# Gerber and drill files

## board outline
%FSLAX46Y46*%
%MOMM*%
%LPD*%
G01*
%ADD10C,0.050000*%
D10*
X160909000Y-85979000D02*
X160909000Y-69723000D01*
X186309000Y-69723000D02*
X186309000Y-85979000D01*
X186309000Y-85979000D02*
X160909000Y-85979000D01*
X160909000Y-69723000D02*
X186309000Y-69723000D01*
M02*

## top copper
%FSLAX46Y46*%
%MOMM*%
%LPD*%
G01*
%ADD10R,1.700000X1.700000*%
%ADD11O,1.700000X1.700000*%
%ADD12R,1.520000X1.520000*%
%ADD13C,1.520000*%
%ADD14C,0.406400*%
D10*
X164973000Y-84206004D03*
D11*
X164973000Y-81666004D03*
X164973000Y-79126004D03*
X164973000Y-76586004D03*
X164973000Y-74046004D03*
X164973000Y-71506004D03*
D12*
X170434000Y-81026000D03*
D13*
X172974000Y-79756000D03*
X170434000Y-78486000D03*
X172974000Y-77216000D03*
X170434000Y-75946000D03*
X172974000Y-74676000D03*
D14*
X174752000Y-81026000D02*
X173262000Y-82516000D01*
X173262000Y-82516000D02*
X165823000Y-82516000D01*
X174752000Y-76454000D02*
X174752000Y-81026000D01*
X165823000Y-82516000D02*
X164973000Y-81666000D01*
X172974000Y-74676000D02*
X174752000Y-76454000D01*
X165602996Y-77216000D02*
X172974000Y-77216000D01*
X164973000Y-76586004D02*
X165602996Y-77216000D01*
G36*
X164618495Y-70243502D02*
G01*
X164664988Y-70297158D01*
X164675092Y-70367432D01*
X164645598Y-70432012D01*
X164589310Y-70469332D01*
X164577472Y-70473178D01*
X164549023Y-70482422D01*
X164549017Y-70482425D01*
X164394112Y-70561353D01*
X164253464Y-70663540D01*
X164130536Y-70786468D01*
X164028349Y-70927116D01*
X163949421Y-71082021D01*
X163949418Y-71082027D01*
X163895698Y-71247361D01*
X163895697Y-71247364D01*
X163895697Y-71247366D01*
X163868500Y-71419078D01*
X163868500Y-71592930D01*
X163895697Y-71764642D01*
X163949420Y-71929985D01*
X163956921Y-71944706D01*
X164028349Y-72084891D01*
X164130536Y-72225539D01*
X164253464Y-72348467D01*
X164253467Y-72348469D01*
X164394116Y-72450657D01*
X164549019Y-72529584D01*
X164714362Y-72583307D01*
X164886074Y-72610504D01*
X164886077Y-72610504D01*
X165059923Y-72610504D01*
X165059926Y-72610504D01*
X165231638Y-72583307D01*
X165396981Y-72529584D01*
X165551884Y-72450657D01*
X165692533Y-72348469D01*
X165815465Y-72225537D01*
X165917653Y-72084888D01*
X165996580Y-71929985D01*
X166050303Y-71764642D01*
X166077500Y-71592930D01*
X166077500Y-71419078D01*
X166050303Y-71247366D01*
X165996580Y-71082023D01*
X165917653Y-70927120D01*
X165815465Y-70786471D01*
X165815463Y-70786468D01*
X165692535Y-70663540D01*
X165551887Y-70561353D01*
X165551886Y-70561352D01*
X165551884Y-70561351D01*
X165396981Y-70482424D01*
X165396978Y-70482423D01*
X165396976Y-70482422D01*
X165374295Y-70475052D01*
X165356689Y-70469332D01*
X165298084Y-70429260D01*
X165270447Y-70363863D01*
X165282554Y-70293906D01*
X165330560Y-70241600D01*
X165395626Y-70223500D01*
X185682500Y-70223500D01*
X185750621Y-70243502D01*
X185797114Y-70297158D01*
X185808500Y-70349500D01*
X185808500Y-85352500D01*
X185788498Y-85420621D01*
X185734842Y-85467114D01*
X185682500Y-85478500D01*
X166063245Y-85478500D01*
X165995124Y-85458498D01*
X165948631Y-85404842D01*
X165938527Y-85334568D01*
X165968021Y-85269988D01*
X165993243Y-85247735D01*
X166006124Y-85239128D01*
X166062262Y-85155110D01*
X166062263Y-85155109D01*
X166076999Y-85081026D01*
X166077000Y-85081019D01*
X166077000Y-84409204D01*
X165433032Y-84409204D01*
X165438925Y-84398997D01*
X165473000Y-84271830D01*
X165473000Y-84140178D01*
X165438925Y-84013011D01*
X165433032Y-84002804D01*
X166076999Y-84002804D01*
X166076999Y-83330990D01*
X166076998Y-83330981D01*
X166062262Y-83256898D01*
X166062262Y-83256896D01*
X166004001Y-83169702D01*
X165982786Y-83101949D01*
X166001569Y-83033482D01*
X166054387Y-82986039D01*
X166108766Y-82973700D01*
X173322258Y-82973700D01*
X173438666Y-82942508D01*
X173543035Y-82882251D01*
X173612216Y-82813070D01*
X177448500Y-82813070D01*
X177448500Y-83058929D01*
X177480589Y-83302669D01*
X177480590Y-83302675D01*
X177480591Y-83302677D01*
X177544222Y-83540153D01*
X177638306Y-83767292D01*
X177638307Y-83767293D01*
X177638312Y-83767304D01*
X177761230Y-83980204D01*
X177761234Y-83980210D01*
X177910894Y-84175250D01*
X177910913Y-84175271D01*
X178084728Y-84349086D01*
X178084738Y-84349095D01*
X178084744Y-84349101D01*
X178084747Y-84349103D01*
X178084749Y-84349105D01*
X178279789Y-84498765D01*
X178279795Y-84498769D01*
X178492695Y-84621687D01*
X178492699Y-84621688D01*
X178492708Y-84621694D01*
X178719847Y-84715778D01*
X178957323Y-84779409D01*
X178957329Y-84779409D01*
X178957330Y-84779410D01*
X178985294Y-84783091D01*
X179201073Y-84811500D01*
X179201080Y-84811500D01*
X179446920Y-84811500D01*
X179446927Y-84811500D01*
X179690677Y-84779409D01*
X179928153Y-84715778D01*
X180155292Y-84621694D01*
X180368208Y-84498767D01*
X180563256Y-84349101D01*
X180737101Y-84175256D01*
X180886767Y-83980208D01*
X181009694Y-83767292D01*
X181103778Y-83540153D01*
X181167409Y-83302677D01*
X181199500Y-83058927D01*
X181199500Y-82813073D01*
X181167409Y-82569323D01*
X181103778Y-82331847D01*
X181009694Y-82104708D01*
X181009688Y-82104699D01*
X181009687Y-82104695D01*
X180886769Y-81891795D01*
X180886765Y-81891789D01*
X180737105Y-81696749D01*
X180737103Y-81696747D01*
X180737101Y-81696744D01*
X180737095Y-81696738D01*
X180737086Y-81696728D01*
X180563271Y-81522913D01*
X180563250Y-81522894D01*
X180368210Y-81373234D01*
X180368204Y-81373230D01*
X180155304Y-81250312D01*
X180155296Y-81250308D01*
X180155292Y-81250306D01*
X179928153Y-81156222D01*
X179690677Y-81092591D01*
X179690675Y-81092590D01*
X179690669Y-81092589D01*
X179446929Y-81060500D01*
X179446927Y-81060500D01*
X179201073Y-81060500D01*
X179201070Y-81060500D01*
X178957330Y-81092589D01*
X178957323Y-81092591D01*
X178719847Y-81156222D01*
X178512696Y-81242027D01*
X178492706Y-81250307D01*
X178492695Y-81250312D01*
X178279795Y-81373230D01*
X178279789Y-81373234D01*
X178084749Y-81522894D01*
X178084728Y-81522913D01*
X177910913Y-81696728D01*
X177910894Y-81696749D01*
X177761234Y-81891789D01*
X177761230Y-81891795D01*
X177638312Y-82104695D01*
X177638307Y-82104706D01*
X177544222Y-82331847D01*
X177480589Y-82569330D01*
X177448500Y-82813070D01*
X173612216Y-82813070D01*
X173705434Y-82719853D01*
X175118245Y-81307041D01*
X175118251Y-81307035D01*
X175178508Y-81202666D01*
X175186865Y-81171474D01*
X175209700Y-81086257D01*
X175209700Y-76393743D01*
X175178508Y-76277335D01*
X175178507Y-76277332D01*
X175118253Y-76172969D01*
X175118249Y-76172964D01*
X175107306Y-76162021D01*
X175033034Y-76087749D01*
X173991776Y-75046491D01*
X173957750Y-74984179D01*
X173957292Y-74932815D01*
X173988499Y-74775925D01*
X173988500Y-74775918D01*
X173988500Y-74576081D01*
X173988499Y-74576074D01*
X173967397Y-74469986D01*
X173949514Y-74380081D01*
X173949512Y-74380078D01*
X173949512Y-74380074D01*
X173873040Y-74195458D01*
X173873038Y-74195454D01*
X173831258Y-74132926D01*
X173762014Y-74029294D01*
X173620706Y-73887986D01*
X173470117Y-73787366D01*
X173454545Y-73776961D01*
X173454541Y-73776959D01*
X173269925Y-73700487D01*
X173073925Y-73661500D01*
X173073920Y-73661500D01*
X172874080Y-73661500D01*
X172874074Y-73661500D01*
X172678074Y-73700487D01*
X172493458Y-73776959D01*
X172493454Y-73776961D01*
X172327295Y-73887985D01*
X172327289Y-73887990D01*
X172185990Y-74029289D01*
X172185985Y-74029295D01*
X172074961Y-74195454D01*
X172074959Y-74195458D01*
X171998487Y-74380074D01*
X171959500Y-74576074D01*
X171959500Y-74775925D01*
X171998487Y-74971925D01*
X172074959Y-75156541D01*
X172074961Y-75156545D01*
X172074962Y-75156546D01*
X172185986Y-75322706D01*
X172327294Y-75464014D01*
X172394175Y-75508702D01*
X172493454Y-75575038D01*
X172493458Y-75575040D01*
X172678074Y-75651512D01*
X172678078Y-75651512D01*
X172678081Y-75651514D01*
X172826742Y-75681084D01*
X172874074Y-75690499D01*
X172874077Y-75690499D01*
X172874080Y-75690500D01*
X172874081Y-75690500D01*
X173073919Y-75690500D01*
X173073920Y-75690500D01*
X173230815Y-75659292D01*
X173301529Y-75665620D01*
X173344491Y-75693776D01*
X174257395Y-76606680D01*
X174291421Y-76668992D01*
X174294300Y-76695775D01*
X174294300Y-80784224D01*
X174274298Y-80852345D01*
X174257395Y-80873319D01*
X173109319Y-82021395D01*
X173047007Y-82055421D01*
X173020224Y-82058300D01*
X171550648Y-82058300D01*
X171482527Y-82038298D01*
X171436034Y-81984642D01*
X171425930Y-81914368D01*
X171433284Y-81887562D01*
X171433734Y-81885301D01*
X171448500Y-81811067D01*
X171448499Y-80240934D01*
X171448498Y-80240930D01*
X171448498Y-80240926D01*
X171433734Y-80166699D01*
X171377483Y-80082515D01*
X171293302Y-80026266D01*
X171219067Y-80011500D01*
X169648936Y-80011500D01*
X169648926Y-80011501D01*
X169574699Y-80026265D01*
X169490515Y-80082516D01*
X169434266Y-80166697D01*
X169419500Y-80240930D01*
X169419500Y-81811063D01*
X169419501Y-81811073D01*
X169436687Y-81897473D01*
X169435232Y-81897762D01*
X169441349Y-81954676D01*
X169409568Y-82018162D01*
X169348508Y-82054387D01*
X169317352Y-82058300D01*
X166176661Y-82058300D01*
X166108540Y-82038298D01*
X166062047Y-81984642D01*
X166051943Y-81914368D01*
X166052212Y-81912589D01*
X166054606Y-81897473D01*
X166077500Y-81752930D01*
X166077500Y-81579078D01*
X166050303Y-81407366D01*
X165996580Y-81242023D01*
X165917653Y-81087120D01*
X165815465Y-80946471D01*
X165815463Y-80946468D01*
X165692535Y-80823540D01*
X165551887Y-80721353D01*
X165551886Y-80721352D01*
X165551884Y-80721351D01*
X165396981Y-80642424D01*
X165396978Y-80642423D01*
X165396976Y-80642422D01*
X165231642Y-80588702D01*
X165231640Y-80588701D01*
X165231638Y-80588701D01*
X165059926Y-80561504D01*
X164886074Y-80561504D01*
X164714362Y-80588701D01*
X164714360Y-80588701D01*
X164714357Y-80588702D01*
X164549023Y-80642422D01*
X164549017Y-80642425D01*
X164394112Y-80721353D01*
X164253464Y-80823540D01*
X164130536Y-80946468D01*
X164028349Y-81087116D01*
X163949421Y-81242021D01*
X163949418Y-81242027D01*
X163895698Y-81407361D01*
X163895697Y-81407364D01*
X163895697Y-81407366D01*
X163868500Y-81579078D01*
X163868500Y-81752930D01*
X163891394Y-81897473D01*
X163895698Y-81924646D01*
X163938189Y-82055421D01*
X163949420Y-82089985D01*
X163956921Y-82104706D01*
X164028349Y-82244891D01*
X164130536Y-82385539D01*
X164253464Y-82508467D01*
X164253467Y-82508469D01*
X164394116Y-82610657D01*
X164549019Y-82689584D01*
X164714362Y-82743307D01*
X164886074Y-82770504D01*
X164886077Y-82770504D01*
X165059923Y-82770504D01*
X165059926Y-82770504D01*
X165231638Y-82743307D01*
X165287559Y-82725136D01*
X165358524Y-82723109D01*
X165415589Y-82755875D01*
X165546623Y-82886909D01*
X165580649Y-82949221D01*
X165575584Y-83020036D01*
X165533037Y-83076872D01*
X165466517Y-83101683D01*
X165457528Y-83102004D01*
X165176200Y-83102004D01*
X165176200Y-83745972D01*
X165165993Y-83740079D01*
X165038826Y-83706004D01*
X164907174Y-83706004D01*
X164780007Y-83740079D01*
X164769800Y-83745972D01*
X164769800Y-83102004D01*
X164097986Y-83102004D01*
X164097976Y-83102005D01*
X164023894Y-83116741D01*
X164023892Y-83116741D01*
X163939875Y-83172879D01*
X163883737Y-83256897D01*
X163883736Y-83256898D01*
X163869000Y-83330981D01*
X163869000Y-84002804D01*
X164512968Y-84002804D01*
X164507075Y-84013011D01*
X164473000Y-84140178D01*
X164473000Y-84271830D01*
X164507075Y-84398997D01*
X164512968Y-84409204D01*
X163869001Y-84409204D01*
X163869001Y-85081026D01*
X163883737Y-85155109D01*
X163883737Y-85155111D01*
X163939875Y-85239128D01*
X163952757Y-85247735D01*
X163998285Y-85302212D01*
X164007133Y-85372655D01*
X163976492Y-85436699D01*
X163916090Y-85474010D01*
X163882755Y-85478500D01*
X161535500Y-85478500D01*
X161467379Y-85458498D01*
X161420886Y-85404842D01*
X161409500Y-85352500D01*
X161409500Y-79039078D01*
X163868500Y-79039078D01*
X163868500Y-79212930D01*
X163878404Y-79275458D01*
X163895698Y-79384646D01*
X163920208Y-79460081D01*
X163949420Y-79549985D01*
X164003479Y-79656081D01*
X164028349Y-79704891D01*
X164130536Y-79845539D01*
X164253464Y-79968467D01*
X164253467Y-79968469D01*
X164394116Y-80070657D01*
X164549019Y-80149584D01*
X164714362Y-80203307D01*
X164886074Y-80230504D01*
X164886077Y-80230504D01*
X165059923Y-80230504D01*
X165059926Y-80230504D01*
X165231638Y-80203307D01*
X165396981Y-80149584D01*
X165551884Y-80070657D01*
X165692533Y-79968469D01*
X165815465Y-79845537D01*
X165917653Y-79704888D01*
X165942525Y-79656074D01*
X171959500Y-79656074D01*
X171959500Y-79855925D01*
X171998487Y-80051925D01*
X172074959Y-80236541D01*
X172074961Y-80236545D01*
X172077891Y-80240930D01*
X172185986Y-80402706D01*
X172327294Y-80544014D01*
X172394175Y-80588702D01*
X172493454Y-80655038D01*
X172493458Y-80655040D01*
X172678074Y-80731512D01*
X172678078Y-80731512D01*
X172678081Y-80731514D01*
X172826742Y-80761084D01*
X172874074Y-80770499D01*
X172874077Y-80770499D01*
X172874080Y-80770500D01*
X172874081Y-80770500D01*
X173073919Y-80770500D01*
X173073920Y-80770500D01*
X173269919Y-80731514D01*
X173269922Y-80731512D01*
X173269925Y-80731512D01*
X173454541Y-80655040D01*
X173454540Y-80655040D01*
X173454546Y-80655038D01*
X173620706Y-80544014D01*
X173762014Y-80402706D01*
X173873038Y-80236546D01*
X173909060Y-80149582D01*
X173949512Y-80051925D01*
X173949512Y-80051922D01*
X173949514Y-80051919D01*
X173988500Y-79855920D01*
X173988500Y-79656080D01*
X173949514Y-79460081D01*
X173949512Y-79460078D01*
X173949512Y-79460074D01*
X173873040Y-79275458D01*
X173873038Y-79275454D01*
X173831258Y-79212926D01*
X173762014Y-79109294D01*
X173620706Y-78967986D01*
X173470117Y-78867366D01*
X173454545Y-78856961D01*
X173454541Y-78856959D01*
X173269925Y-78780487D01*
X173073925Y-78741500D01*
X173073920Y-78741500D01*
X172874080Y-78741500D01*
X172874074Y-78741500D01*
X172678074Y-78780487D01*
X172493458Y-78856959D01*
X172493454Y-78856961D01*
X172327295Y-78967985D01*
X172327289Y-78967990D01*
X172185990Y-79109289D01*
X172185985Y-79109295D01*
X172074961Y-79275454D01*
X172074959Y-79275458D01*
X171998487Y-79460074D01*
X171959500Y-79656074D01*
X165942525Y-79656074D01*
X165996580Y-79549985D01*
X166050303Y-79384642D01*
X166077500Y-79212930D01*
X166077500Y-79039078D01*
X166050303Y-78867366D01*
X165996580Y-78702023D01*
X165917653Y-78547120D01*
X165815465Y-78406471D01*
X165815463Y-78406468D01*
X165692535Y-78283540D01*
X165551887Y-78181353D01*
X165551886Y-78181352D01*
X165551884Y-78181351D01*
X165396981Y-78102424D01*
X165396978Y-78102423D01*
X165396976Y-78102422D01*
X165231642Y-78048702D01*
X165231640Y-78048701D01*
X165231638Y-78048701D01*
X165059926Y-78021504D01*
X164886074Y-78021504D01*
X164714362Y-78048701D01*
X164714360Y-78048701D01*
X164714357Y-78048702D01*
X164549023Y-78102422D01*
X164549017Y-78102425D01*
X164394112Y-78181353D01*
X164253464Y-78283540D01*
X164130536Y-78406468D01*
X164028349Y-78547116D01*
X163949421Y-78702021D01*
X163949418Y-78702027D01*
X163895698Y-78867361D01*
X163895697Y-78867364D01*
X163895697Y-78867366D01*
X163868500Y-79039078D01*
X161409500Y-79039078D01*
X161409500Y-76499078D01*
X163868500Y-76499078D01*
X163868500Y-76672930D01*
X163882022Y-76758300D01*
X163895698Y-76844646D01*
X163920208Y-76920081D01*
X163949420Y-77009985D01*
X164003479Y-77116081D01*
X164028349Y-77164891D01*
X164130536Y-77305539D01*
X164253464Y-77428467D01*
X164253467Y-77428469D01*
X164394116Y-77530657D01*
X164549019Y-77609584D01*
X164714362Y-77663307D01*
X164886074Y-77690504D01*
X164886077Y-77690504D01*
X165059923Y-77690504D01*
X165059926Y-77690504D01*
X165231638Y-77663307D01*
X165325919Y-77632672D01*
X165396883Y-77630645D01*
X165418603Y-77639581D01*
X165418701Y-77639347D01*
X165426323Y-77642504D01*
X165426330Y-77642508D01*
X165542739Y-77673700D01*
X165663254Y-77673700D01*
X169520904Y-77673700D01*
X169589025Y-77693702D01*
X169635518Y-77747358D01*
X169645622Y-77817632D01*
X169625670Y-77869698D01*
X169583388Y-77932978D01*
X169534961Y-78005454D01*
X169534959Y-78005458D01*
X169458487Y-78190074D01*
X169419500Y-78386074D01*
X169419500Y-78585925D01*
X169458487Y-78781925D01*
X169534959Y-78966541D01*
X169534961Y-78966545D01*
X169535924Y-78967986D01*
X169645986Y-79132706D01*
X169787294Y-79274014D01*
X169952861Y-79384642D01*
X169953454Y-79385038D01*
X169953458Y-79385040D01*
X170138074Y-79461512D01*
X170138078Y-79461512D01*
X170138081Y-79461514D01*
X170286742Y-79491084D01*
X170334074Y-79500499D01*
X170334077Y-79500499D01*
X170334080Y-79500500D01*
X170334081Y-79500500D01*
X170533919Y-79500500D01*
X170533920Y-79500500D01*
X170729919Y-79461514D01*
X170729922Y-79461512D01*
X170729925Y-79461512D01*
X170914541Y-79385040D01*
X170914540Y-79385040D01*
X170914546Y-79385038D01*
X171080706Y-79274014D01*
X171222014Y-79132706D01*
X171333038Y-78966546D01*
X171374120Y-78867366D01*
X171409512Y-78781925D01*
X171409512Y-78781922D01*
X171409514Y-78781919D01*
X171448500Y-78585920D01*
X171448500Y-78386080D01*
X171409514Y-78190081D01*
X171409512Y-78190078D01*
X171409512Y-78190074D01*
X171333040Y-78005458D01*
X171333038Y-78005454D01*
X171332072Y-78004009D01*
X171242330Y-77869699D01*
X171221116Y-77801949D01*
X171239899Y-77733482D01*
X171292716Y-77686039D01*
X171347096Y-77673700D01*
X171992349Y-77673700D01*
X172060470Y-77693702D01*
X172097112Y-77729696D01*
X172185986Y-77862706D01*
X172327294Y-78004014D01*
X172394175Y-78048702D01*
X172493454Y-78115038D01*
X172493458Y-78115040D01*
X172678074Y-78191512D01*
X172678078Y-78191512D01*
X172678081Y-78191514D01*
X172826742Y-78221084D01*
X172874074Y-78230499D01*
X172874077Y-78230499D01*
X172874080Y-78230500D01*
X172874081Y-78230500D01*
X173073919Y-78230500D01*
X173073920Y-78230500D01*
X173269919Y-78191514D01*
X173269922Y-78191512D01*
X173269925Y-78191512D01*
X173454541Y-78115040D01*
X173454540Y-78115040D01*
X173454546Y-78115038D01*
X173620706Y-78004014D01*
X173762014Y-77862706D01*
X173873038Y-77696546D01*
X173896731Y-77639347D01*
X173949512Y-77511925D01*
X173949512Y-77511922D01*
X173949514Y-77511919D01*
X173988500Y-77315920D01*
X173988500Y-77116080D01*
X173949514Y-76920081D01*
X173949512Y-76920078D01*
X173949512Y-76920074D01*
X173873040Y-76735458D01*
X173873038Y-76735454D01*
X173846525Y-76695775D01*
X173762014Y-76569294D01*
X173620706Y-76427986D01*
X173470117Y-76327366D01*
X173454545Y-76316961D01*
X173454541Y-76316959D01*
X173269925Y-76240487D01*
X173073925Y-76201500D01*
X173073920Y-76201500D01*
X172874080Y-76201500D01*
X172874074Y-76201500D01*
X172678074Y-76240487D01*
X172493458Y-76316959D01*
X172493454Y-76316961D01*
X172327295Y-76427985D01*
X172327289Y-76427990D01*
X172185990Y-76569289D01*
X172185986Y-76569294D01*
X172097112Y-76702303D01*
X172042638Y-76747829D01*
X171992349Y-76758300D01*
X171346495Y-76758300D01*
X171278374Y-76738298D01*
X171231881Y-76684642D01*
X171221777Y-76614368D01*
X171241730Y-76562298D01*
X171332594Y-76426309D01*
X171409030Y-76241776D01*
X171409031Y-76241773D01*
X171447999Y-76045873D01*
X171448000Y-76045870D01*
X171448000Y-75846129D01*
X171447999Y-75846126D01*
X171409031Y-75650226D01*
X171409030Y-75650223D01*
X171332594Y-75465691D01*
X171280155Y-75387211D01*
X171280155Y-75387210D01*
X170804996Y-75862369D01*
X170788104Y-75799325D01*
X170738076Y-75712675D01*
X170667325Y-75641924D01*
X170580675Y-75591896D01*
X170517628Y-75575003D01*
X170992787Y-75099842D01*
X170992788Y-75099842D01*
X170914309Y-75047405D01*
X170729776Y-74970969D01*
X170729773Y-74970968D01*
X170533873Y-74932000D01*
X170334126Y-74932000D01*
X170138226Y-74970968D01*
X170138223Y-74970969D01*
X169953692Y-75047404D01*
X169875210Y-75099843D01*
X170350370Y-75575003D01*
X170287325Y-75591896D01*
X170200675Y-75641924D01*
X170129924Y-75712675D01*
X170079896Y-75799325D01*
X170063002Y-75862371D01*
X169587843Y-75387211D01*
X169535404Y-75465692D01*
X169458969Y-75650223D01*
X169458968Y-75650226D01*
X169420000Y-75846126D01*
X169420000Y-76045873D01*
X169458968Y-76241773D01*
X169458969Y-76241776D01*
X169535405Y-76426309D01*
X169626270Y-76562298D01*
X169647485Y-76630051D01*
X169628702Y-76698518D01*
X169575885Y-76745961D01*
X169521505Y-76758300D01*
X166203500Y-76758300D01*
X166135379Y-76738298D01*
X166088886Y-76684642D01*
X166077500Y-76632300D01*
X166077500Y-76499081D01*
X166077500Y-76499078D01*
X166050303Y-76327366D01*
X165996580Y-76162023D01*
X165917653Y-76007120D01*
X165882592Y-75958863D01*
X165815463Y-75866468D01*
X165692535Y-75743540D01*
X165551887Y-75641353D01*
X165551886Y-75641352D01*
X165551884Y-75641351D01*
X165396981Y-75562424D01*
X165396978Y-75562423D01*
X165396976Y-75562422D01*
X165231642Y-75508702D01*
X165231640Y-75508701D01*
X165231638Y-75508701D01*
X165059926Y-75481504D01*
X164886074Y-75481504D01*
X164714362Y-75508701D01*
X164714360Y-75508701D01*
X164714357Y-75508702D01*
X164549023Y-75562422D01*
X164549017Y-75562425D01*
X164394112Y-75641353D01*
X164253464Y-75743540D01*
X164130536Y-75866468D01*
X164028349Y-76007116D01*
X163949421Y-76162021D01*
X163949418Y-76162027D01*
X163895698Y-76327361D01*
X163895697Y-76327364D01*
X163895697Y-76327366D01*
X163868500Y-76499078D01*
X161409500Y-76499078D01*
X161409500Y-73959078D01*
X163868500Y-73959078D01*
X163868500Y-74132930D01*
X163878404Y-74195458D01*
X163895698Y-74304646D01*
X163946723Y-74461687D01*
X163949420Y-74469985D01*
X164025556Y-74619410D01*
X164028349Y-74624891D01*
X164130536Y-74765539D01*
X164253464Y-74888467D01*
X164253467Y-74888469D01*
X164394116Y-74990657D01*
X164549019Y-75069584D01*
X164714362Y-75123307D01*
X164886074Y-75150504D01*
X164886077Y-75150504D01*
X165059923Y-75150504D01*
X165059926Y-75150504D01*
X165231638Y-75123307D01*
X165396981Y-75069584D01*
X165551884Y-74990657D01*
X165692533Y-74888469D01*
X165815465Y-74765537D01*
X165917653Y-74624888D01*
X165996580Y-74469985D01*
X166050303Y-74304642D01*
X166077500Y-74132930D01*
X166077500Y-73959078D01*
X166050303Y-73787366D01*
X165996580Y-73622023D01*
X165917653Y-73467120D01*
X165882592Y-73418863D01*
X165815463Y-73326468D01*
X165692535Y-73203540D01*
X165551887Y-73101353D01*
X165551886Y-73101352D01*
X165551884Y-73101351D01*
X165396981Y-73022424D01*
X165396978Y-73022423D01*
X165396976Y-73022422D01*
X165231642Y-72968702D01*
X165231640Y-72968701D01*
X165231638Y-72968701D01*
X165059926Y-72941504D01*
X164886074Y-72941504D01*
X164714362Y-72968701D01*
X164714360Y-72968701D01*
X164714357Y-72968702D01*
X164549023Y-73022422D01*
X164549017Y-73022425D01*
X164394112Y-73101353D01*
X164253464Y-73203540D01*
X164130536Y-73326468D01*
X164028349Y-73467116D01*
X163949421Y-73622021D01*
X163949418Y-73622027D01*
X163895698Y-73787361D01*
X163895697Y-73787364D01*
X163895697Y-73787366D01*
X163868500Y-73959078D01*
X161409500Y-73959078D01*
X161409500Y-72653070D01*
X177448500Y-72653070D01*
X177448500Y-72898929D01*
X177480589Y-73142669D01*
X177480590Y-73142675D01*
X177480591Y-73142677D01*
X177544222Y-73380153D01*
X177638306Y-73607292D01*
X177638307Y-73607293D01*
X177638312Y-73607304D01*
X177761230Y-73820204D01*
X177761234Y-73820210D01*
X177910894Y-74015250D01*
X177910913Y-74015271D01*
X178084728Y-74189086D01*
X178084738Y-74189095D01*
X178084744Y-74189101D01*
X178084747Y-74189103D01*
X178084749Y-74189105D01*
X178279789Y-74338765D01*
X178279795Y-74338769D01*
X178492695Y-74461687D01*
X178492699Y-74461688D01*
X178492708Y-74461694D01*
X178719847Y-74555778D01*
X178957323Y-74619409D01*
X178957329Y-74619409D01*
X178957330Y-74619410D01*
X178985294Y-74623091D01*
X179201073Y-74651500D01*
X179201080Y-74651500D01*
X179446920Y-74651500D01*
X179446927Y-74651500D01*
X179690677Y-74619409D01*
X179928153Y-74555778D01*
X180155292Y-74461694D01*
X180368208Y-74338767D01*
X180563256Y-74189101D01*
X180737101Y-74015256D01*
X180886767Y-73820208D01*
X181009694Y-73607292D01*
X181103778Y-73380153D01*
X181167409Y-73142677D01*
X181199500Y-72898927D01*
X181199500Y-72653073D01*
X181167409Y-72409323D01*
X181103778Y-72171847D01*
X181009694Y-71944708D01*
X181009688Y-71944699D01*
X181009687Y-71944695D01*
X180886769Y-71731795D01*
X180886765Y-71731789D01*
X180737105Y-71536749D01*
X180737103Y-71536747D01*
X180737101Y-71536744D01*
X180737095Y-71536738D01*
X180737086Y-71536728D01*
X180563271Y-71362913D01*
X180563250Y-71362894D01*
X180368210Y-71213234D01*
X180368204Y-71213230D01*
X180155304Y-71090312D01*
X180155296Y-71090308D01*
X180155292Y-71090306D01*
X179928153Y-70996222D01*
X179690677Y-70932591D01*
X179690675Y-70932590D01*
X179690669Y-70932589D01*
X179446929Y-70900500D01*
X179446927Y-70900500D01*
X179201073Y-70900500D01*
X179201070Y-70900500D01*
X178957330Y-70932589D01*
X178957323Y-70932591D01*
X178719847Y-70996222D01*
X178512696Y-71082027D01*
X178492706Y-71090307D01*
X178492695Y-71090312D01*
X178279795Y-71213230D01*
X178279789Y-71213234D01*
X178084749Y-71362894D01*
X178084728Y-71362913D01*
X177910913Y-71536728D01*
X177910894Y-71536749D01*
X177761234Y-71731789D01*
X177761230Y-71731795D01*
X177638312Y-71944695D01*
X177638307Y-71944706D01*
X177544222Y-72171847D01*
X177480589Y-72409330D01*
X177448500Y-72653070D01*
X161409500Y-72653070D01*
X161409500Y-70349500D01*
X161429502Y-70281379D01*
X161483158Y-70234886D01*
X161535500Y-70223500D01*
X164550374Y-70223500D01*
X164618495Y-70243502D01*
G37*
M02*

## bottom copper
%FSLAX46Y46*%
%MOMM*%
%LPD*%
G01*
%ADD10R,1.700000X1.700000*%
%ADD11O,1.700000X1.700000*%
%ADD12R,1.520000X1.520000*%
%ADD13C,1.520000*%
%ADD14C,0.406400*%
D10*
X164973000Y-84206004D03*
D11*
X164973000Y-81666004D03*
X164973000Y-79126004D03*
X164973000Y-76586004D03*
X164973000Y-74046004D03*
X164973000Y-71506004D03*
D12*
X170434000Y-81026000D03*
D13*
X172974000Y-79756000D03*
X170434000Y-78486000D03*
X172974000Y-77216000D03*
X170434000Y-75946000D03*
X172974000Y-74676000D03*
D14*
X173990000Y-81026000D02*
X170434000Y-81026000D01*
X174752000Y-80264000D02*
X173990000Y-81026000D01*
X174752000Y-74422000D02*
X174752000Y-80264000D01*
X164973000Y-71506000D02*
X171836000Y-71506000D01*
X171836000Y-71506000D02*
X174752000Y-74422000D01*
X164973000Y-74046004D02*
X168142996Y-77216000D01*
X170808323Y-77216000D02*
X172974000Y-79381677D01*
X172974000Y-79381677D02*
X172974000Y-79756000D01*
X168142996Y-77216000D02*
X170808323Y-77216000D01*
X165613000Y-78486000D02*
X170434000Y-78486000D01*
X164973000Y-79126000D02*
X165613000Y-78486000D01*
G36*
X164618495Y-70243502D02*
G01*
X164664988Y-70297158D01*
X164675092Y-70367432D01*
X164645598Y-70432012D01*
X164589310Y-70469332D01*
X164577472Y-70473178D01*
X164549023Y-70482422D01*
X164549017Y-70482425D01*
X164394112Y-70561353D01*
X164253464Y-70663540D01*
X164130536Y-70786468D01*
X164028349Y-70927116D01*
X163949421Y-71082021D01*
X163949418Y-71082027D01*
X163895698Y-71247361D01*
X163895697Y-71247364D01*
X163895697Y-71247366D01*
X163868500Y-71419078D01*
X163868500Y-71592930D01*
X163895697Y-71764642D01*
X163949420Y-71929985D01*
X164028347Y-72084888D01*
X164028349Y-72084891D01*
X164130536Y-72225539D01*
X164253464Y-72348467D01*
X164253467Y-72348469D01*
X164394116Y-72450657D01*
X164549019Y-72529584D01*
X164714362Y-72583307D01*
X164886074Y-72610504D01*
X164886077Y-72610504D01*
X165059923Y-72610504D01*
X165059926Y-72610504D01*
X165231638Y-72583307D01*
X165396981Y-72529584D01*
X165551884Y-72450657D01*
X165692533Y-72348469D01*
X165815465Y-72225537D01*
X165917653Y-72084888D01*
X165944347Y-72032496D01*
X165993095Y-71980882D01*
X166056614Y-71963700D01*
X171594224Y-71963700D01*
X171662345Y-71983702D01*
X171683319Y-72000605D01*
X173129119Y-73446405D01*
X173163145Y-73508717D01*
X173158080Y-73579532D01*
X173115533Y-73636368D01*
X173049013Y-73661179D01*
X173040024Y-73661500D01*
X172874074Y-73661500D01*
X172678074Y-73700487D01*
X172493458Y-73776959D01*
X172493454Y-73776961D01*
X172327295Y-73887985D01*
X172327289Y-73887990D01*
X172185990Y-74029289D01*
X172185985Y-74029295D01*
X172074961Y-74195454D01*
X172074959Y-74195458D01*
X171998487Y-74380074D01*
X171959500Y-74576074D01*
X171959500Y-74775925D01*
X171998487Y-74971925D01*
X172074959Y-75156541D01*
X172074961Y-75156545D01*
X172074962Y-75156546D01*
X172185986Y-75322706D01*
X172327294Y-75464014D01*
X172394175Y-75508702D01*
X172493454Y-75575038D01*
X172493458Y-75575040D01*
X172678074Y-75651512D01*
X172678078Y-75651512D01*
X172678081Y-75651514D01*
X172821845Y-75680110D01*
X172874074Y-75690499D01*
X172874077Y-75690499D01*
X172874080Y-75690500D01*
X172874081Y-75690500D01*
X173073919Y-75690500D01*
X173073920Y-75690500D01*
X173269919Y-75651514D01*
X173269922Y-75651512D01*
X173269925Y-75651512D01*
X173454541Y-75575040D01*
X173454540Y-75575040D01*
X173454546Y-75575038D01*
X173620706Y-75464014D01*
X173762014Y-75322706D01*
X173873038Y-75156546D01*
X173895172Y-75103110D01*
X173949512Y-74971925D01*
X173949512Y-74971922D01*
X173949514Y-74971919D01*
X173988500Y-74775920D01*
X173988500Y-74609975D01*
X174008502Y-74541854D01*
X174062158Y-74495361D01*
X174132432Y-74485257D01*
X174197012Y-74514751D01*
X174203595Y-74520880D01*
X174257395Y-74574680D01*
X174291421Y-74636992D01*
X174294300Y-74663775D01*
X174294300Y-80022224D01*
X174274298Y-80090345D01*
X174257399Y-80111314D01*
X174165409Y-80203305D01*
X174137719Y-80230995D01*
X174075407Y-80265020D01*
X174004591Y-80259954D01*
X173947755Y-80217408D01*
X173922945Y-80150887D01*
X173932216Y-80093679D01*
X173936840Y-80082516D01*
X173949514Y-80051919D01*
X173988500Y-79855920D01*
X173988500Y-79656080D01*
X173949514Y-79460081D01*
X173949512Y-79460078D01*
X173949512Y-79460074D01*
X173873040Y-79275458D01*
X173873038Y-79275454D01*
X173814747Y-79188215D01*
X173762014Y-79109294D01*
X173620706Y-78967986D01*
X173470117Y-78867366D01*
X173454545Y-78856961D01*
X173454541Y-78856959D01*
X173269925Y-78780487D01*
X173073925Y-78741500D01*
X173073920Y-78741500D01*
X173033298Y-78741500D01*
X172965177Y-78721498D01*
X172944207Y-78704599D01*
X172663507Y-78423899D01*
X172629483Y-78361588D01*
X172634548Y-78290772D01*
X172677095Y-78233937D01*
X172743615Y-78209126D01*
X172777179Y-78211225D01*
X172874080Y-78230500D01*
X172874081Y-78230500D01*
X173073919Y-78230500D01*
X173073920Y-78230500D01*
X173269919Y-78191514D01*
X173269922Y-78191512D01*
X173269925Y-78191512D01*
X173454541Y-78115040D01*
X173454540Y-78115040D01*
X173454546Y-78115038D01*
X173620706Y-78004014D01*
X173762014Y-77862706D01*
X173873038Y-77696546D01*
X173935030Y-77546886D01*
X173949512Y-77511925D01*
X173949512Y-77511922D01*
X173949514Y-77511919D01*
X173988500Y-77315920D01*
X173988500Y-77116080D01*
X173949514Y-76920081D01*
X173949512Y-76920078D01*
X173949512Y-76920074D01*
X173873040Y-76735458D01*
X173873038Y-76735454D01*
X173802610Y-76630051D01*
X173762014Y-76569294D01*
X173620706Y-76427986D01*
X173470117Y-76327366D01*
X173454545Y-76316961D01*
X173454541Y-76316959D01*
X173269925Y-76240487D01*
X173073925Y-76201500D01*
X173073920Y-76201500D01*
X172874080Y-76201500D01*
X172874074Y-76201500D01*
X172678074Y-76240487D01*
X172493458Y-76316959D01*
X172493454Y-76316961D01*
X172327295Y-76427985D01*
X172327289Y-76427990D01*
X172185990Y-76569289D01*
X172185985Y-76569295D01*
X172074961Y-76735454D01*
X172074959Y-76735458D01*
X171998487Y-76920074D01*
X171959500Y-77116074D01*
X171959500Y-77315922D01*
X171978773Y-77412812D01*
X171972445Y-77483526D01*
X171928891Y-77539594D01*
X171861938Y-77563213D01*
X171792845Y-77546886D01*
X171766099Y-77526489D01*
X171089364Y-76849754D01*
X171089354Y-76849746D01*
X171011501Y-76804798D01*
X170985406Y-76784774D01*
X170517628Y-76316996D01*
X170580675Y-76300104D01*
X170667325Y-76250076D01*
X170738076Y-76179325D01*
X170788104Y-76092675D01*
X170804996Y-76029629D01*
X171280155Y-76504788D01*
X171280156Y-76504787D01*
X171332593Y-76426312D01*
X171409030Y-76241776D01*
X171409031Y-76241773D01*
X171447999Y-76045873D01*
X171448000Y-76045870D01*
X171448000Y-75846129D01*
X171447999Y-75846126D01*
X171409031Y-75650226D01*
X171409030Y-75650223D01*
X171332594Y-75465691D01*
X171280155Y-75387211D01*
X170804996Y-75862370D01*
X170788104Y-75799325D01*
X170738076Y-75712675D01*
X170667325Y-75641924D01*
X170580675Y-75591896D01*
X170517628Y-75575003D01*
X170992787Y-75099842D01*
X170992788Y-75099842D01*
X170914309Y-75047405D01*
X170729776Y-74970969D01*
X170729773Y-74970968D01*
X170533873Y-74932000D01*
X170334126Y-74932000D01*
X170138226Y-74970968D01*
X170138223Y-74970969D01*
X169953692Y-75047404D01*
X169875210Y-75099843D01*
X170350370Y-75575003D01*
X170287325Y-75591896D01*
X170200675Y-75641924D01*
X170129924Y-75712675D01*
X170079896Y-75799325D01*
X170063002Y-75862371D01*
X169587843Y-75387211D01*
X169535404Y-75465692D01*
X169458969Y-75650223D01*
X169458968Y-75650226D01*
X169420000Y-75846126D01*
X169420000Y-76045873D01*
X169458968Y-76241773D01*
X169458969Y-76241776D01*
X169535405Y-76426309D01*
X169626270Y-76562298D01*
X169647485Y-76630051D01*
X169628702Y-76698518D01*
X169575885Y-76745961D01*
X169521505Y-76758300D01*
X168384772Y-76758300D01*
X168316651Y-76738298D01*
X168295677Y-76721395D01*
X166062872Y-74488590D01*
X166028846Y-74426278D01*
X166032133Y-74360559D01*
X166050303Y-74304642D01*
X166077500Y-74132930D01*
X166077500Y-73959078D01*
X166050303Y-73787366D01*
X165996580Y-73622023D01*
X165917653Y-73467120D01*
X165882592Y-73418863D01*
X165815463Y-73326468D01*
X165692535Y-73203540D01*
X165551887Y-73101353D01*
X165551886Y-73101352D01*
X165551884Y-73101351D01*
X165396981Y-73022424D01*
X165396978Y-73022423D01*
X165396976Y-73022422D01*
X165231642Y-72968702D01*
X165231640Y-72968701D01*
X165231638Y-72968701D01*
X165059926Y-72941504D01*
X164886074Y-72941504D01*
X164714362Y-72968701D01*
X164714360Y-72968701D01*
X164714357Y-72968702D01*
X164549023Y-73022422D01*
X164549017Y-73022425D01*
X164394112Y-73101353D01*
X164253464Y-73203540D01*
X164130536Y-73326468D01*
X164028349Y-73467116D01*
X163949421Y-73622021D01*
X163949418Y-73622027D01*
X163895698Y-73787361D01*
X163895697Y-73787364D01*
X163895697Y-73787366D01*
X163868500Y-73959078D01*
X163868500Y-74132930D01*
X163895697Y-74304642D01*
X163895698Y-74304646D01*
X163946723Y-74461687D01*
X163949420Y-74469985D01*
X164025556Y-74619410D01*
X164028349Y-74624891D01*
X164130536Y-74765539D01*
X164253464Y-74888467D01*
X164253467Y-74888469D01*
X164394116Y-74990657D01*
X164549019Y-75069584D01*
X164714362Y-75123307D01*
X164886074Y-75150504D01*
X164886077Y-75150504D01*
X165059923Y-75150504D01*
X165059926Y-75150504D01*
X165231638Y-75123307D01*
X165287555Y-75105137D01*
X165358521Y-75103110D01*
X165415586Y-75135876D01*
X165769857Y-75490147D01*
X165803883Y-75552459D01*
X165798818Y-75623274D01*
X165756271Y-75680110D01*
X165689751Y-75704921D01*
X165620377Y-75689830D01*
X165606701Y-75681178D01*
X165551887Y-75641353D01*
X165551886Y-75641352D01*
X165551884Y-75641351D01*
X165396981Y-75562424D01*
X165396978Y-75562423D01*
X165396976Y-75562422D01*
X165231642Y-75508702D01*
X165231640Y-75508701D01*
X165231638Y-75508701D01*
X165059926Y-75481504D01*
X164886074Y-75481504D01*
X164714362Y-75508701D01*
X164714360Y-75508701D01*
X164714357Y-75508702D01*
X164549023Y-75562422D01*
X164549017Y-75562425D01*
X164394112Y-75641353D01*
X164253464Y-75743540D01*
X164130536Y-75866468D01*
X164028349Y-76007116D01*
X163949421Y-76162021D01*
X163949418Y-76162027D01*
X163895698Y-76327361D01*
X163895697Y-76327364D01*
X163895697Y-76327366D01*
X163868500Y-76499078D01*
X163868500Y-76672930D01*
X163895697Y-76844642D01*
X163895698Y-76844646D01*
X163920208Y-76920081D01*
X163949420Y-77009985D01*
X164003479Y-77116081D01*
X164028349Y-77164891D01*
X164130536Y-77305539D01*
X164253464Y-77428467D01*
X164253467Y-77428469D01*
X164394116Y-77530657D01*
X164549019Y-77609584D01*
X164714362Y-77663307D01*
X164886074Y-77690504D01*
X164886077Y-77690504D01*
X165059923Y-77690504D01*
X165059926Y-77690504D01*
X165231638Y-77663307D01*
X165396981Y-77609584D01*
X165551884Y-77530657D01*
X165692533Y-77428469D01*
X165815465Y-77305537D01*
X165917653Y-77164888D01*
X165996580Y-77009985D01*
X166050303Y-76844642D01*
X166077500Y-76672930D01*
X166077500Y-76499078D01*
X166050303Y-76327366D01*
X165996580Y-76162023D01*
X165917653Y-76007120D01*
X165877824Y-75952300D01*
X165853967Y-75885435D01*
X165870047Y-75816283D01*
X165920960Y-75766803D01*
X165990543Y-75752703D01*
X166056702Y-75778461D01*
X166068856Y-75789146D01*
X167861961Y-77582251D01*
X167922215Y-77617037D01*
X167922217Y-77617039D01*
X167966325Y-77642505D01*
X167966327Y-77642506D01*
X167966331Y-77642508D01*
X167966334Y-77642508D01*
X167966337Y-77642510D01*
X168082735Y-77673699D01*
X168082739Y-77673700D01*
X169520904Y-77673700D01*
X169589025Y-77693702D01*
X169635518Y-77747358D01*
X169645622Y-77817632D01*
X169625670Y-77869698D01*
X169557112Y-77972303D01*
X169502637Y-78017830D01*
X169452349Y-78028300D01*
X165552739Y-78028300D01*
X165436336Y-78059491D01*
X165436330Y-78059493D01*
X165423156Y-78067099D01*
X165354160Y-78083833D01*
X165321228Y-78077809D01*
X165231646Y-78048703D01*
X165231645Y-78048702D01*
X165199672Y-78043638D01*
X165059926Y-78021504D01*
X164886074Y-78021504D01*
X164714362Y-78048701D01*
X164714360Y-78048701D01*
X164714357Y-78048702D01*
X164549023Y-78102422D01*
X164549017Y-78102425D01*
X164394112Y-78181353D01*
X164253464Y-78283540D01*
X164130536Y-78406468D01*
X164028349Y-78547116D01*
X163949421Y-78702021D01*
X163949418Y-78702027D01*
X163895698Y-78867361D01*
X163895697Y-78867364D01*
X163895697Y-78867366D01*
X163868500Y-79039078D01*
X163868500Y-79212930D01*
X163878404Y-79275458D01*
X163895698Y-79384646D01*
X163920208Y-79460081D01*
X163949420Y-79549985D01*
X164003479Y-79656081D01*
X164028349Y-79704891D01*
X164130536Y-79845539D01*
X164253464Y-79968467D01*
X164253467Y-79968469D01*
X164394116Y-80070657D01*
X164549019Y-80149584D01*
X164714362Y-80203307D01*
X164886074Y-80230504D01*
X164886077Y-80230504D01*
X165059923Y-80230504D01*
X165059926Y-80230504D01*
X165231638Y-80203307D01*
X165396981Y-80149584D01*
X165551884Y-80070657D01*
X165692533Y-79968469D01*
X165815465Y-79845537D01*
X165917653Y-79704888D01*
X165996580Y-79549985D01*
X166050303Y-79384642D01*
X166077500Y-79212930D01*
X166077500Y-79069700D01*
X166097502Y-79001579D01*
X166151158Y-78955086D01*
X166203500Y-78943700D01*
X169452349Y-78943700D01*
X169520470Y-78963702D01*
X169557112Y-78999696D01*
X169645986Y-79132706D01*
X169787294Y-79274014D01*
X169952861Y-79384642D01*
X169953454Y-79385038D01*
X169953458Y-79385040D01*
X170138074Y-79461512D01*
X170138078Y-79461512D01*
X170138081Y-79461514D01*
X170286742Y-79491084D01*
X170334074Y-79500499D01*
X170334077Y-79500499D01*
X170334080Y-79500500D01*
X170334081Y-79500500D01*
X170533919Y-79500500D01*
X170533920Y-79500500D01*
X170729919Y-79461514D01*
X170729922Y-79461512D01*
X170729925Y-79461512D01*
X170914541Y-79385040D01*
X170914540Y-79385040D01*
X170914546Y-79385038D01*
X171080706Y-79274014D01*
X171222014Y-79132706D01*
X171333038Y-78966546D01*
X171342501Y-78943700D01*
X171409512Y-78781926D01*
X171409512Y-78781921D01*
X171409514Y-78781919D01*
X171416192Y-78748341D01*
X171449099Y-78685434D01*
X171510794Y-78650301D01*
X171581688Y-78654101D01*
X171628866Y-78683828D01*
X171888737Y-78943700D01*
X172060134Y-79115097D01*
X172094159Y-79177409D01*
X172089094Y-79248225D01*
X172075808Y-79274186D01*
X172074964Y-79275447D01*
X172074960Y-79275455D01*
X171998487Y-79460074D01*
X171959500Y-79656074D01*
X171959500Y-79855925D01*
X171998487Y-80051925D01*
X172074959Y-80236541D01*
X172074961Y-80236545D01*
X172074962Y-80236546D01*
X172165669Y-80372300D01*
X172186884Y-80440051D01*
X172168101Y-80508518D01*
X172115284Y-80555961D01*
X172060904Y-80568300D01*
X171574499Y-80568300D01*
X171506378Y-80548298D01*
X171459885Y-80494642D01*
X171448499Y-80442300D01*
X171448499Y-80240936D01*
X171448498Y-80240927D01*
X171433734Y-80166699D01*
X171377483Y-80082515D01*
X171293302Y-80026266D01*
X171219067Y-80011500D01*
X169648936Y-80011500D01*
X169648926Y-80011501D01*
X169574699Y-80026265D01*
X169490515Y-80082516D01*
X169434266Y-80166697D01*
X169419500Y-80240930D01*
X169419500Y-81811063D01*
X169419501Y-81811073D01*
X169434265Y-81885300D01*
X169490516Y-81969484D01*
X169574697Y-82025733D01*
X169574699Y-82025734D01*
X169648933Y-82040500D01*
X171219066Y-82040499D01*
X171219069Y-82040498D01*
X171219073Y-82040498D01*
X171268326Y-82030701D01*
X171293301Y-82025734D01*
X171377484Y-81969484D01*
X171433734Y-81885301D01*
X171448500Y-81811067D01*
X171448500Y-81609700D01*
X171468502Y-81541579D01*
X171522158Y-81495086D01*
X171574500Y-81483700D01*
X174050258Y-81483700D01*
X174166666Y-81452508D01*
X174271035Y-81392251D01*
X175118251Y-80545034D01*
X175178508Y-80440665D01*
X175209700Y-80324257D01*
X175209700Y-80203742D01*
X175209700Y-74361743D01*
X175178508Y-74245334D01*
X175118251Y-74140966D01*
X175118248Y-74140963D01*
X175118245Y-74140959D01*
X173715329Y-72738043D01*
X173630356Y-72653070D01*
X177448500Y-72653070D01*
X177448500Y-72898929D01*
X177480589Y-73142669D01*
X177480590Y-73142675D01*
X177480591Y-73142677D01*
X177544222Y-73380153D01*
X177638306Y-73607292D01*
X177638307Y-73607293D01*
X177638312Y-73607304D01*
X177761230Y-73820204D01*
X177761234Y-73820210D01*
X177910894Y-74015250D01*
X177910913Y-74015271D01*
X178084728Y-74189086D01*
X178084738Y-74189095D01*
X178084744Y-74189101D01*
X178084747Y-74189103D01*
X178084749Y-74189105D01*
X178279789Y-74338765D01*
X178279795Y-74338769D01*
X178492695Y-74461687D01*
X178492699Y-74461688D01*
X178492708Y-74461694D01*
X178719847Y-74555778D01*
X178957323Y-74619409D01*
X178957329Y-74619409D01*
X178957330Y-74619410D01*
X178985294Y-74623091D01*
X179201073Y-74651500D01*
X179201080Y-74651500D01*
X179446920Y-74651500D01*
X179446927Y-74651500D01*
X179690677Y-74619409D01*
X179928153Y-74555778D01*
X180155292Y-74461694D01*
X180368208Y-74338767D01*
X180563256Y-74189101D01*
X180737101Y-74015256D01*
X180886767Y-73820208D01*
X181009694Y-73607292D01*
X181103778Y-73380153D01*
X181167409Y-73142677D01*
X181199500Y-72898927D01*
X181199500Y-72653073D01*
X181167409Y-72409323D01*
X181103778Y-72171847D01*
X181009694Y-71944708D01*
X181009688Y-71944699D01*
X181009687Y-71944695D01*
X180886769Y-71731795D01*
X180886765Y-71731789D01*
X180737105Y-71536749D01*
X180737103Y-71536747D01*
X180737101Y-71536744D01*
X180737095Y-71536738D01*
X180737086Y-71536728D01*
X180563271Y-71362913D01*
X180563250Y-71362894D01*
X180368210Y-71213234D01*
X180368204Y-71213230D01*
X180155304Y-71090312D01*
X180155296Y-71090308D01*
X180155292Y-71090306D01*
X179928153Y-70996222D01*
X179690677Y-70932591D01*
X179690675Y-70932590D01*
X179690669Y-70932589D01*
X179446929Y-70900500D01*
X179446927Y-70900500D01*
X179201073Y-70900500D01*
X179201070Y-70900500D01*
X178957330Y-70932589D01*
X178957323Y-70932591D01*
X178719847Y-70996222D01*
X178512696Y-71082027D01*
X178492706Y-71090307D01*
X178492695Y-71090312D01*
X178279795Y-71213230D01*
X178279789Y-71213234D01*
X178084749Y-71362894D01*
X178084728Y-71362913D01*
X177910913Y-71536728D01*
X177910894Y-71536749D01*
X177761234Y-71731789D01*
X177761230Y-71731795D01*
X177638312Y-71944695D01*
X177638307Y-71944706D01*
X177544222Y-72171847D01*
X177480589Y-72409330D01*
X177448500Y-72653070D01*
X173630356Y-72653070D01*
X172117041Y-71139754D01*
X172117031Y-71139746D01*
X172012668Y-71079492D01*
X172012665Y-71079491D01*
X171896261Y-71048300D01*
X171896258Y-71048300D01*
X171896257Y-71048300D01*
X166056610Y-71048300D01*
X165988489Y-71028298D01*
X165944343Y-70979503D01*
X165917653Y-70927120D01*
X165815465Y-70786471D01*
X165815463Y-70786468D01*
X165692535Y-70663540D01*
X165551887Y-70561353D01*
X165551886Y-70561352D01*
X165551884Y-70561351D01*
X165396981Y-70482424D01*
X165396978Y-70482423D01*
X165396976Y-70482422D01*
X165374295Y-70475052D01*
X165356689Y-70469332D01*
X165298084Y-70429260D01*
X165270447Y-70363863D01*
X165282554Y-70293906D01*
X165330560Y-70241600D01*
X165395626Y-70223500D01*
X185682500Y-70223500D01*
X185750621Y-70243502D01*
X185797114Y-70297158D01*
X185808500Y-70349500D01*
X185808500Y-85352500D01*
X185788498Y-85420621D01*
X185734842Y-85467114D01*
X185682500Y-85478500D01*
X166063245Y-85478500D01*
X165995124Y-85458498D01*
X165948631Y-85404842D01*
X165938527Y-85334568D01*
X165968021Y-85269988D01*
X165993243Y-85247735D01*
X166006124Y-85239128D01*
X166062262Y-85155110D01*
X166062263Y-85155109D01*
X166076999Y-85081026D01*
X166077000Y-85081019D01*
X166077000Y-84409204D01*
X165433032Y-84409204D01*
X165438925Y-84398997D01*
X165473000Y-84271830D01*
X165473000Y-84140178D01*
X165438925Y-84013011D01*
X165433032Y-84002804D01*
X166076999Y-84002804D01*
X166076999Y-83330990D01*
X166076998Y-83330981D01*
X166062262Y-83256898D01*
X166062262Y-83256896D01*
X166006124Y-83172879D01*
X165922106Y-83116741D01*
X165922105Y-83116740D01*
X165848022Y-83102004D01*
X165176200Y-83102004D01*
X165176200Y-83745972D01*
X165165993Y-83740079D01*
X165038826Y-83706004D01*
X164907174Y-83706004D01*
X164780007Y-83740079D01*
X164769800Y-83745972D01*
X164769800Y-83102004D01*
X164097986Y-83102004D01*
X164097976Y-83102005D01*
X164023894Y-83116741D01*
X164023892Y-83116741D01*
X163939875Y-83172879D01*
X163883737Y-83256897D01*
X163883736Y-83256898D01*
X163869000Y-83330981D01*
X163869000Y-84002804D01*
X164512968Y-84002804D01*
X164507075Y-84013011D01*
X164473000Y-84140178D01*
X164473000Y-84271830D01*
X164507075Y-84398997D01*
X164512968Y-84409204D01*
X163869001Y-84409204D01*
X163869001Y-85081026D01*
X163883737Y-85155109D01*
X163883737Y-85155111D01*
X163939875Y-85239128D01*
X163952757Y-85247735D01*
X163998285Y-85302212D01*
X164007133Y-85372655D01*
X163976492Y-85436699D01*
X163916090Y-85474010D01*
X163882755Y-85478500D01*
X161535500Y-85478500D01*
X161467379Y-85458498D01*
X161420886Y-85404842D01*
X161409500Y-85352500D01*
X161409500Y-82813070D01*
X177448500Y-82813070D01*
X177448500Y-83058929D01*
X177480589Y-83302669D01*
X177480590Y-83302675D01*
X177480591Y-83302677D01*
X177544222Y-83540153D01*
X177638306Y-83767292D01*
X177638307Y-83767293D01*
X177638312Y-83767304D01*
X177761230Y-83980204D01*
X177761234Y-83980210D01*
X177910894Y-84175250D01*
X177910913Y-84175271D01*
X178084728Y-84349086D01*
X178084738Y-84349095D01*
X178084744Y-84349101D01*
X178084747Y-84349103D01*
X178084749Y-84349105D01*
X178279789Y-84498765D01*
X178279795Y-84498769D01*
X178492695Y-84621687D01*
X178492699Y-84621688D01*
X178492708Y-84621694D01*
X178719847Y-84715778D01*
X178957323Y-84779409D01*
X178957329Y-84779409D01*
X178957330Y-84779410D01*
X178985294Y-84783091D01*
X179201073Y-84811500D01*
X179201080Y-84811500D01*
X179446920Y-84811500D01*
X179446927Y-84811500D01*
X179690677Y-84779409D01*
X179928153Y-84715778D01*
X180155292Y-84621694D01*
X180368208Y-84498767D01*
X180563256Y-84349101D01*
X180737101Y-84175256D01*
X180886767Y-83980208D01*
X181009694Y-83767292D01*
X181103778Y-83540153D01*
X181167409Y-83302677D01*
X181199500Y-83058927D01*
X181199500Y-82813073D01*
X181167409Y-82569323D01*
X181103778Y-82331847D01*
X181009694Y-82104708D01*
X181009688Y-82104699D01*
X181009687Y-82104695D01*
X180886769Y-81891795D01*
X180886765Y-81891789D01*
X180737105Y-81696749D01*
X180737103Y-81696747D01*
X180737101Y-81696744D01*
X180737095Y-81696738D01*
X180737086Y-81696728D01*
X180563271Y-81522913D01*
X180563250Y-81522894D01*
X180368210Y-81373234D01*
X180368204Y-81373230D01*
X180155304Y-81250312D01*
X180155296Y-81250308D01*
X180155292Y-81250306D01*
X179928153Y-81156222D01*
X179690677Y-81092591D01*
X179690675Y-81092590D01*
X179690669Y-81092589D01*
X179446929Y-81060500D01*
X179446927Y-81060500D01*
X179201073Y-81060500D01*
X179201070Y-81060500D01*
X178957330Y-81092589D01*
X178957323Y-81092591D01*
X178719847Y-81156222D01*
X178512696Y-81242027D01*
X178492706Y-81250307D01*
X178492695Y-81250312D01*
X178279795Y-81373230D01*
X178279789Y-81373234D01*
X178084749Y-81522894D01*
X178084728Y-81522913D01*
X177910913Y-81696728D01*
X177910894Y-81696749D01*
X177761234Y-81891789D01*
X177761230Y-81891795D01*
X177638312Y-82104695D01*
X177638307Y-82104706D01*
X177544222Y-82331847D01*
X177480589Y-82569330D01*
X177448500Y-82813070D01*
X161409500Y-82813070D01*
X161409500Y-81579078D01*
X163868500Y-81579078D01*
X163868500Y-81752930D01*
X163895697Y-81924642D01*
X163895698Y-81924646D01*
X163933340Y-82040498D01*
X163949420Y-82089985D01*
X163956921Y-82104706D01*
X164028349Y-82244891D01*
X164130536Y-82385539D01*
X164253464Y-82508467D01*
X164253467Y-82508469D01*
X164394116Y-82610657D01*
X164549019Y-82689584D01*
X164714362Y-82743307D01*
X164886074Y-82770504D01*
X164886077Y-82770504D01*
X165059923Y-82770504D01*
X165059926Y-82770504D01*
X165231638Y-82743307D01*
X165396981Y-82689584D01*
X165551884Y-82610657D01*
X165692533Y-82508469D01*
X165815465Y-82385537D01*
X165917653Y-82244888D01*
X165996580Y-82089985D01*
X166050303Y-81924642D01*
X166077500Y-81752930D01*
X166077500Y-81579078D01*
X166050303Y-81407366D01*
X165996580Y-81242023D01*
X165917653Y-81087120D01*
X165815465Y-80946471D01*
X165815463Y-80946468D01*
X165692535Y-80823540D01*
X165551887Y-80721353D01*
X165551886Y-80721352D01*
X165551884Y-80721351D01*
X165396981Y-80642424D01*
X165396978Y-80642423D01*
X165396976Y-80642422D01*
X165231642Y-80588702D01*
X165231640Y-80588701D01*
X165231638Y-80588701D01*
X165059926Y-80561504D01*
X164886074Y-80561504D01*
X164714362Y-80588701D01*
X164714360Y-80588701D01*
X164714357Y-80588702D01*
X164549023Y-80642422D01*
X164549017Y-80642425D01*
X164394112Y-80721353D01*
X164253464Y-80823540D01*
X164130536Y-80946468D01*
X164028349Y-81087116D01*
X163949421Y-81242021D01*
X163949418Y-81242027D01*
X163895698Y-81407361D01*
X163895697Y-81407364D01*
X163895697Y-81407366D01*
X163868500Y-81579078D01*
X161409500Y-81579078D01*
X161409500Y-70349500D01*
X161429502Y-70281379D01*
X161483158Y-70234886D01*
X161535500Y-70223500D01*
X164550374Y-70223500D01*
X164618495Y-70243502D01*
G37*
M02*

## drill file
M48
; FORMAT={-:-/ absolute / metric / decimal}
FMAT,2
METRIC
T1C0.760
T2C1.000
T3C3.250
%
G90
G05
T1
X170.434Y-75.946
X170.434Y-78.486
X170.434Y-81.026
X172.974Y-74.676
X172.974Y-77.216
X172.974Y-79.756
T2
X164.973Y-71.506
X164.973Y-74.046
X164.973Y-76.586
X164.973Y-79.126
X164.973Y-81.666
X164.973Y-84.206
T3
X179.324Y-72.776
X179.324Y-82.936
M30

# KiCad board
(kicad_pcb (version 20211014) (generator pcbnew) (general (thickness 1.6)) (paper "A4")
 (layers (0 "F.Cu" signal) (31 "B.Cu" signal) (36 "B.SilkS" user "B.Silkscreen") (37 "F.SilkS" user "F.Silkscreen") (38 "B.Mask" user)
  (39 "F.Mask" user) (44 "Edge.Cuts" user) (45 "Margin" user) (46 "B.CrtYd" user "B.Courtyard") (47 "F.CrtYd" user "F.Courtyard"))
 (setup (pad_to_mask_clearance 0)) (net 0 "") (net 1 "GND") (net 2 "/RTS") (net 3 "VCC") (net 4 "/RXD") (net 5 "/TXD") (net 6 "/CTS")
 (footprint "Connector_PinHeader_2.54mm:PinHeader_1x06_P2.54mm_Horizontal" (layer "F.Cu") (at 164.973 84.206004 180)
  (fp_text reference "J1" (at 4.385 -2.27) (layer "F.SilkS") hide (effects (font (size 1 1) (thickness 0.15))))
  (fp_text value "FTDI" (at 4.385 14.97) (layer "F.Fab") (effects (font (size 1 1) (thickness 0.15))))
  (pad "1" thru_hole rect locked (at 0 0 180) (size 1.7 1.7) (drill 1) (layers *.Cu *.Mask) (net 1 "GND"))
  (pad "2" thru_hole oval locked (at 0 2.54 180) (size 1.7 1.7) (drill 1) (layers *.Cu *.Mask) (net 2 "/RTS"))
  (pad "3" thru_hole oval locked (at 0 5.08 180) (size 1.7 1.7) (drill 1) (layers *.Cu *.Mask) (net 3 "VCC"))
  (pad "4" thru_hole oval locked (at 0 7.62 180) (size 1.7 1.7) (drill 1) (layers *.Cu *.Mask) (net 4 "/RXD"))
  (pad "5" thru_hole oval locked (at 0 10.16 180) (size 1.7 1.7) (drill 1) (layers *.Cu *.Mask) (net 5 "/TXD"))
  (pad "6" thru_hole oval locked (at 0 12.7 180) (size 1.7 1.7) (drill 1) (layers *.Cu *.Mask) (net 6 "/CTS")))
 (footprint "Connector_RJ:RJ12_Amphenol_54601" (layer "F.Cu") (at 170.434 81.026 90)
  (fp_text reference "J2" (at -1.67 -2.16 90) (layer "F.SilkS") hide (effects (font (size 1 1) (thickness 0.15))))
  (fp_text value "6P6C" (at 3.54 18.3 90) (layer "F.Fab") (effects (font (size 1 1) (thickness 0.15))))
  (pad "" np_thru_hole circle locked (at 8.25 8.89 90) (size 3.25 3.25) (drill 3.25) (layers *.Cu *.Mask))
  (pad "" np_thru_hole circle locked (at -1.91 8.89 90) (size 3.25 3.25) (drill 3.25) (layers *.Cu *.Mask))
  (pad "1" thru_hole rect locked (at 0 0 90) (size 1.52 1.52) (drill 0.76) (layers *.Cu *.Mask) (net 6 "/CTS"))
  (pad "2" thru_hole circle locked (at 1.27 2.54 90) (size 1.52 1.52) (drill 0.76) (layers *.Cu *.Mask) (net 5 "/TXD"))
  (pad "3" thru_hole circle locked (at 2.54 0 90) (size 1.52 1.52) (drill 0.76) (layers *.Cu *.Mask) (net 3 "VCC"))
  (pad "4" thru_hole circle locked (at 3.81 2.54 90) (size 1.52 1.52) (drill 0.76) (layers *.Cu *.Mask) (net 4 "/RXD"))
  (pad "5" thru_hole circle locked (at 5.08 0 90) (size 1.52 1.52) (drill 0.76) (layers *.Cu *.Mask) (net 1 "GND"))
  (pad "6" thru_hole circle locked (at 6.35 2.54 90) (size 1.52 1.52) (drill 0.76) (layers *.Cu *.Mask) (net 2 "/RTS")))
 (gr_line (start 160.909 85.979) (end 160.909 69.723) (layer "Edge.Cuts") (width 0.05))
 (gr_line (start 186.309 69.723) (end 186.309 85.979) (layer "Edge.Cuts") (width 0.05))
 (gr_line (start 186.309 85.979) (end 160.909 85.979) (layer "Edge.Cuts") (width 0.05))
 (gr_line (start 160.909 69.723) (end 186.309 69.723) (layer "Edge.Cuts") (width 0.05))
 (segment (start 174.752 81.026) (end 173.262 82.516) (width 0.4064) (layer "F.Cu") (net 2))
 (segment (start 173.262 82.516) (end 165.823 82.516) (width 0.4064) (layer "F.Cu") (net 2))
 (segment (start 174.752 76.454) (end 174.752 81.026) (width 0.4064) (layer "F.Cu") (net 2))
 (segment (start 165.823 82.516) (end 164.973 81.666) (width 0.4064) (layer "F.Cu") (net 2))
 (segment (start 172.974 74.676) (end 174.752 76.454) (width 0.4064) (layer "F.Cu") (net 2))
 (segment (start 173.99 81.026) (end 170.434 81.026) (width 0.4064) (layer "B.Cu") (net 6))
 (segment (start 174.752 80.264) (end 173.99 81.026) (width 0.4064) (layer "B.Cu") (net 6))
 (segment (start 174.752 74.422) (end 174.752 80.264) (width 0.4064) (layer "B.Cu") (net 6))
 (segment (start 164.973 71.506) (end 171.836 71.506) (width 0.4064) (layer "B.Cu") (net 6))
 (segment (start 171.836 71.506) (end 174.752 74.422) (width 0.4064) (layer "B.Cu") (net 6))
 (segment (start 164.973 74.046004) (end 168.142996 77.216) (width 0.4064) (layer "B.Cu") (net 5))
 (segment (start 170.808323 77.216) (end 172.974 79.381677) (width 0.4064) (layer "B.Cu") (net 5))
 (segment (start 172.974 79.381677) (end 172.974 79.756) (width 0.4064) (layer "B.Cu") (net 5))
 (segment (start 168.142996 77.216) (end 170.808323 77.216) (width 0.4064) (layer "B.Cu") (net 5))
 (segment (start 165.613 78.486) (end 170.434 78.486) (width 0.4064) (layer "B.Cu") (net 3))
 (segment (start 164.973 79.126) (end 165.613 78.486) (width 0.4064) (layer "B.Cu") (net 3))
 (segment (start 165.602996 77.216) (end 172.974 77.216) (width 0.4064) (layer "F.Cu") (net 4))
 (segment (start 164.973 76.586004) (end 165.602996 77.216) (width 0.4064) (layer "F.Cu") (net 4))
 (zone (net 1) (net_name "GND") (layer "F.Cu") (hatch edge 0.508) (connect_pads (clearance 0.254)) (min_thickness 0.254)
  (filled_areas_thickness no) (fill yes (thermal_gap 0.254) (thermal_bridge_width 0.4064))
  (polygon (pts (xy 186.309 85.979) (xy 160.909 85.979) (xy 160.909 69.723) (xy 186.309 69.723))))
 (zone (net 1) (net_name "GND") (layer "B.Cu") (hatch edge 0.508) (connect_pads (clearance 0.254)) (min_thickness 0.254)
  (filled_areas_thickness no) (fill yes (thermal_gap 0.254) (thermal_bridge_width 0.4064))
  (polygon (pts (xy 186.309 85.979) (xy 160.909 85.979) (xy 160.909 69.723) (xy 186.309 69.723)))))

